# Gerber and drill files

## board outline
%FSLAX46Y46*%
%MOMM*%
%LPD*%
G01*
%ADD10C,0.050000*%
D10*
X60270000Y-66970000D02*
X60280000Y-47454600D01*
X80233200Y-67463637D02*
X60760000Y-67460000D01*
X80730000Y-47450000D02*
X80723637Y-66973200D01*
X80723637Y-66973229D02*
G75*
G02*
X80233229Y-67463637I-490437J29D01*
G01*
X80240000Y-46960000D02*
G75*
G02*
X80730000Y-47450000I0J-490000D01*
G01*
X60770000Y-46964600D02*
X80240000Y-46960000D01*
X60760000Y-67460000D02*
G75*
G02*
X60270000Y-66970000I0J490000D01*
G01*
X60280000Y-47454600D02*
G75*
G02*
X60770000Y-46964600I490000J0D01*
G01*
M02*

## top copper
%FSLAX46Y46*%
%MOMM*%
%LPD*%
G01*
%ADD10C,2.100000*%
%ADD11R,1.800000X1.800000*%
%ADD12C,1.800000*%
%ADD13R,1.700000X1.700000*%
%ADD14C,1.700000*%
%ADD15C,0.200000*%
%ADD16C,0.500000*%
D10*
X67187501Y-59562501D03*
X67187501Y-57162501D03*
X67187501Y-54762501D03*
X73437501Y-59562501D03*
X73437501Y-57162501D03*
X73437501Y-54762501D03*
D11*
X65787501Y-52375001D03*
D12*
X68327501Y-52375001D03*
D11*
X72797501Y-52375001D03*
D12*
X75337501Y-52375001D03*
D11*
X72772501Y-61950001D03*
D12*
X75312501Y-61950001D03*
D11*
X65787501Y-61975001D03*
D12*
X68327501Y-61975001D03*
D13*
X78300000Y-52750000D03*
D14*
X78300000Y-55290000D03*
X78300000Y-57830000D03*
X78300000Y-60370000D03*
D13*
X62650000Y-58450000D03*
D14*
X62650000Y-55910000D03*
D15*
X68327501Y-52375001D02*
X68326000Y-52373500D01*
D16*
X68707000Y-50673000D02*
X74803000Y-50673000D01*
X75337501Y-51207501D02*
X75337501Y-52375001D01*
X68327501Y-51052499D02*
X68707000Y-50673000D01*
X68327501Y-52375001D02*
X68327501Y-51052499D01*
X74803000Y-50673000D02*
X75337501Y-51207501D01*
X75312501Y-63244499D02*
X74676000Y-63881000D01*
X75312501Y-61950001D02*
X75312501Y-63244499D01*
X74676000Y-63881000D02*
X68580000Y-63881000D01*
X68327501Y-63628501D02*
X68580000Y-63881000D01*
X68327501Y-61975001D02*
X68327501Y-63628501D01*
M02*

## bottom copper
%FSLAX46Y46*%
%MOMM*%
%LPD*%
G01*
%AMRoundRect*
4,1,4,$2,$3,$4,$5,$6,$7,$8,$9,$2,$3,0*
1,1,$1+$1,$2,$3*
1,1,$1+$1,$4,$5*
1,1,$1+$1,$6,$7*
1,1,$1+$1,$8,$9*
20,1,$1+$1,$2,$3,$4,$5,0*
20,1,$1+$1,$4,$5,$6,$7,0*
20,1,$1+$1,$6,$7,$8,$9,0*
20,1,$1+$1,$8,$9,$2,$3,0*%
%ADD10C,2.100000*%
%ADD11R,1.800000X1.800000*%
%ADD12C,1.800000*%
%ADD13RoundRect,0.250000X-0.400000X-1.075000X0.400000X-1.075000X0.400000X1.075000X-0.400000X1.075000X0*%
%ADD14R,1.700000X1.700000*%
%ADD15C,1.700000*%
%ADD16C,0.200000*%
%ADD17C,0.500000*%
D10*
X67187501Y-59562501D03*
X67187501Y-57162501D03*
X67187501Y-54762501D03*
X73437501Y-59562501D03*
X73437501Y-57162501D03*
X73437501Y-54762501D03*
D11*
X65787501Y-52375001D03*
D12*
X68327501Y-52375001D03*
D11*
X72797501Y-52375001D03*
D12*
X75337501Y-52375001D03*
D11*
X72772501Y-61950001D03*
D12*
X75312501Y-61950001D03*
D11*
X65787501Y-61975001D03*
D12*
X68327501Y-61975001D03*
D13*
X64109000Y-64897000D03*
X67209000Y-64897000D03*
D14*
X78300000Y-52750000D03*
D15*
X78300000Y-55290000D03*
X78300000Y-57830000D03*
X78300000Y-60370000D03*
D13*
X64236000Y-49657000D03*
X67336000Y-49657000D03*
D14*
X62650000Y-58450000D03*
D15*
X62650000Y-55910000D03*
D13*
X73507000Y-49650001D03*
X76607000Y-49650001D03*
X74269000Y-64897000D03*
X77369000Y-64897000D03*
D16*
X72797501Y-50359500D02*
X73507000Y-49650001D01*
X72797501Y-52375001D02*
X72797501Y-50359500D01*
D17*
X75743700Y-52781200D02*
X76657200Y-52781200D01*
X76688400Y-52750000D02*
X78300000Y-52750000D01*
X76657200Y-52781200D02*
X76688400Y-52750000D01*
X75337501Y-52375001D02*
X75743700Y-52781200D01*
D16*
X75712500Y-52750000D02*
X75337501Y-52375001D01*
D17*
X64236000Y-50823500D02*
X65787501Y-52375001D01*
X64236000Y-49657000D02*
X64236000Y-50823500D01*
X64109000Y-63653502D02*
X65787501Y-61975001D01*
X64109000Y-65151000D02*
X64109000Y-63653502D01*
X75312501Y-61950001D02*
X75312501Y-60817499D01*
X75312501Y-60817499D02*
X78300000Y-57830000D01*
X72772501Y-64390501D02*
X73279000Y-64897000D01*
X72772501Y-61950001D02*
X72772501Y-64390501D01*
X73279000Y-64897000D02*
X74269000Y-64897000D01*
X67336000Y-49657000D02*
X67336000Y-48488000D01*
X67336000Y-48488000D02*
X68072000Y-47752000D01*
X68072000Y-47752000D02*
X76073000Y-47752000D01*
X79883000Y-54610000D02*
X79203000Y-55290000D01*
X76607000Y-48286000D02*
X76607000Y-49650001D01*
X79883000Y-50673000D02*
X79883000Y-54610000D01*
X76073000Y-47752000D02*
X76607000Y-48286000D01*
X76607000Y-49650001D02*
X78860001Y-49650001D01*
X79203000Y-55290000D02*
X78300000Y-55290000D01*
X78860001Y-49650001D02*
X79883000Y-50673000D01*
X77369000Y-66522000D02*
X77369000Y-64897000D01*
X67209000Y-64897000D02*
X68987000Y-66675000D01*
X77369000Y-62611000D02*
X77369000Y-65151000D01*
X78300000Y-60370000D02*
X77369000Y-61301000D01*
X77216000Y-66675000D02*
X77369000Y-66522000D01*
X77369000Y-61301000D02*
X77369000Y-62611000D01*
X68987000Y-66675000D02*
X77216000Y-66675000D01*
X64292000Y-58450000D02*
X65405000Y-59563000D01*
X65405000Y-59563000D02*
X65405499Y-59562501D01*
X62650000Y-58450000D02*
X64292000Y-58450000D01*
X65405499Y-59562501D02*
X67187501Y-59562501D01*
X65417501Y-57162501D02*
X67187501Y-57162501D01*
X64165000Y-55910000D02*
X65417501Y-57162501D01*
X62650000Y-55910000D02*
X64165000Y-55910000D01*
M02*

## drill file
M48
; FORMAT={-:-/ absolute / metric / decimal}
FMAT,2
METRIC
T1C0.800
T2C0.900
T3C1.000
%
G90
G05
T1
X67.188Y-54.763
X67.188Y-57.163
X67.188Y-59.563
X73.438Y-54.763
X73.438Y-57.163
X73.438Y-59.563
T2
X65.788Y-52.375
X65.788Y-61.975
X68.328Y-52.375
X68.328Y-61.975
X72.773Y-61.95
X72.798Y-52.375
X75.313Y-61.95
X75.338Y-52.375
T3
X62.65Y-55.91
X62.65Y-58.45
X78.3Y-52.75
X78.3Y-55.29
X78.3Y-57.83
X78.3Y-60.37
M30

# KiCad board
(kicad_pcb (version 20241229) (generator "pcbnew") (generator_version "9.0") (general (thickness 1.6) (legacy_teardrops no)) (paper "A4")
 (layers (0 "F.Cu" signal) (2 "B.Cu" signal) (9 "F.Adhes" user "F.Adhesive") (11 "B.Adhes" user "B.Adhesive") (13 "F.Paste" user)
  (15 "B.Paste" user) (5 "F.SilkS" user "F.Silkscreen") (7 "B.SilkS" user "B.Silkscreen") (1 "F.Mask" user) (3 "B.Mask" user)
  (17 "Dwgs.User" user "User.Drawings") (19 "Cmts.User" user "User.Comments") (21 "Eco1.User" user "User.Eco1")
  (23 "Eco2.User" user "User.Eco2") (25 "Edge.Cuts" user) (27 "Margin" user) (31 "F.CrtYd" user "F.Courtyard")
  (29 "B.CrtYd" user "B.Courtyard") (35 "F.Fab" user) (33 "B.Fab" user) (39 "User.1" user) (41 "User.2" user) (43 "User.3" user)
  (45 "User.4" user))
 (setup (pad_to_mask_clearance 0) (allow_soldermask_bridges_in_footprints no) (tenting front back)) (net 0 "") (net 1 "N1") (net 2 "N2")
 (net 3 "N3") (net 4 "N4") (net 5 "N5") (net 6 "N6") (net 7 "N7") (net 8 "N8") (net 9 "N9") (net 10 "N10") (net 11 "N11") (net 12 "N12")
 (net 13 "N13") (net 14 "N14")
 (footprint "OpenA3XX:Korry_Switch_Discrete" (layer "F.Cu") (at 76.287501 61.262501)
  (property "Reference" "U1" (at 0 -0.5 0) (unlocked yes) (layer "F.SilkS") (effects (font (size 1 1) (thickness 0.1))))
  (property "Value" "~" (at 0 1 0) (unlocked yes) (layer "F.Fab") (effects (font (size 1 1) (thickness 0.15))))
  (pad "1" thru_hole circle (at -9.1 -1.7) (size 2.1 2.1) (drill 0.8) (layers "*.Cu" "*.Mask") (remove_unused_layers no) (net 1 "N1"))
  (pad "2" thru_hole circle (at -9.1 -4.1) (size 2.1 2.1) (drill 0.8) (layers "*.Cu" "*.Mask") (remove_unused_layers no) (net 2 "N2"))
  (pad "3" thru_hole circle (at -9.1 -6.5) (size 2.1 2.1) (drill 0.8) (layers "*.Cu" "*.Mask") (remove_unused_layers no) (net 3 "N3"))
  (pad "4" thru_hole circle (at -2.85 -1.7) (size 2.1 2.1) (drill 0.8) (layers "*.Cu" "*.Mask") (remove_unused_layers no) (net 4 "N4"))
  (pad "5" thru_hole circle (at -2.85 -4.1) (size 2.1 2.1) (drill 0.8) (layers "*.Cu" "*.Mask") (remove_unused_layers no) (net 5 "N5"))
  (pad "6" thru_hole circle (at -2.85 -6.5) (size 2.1 2.1) (drill 0.8) (layers "*.Cu" "*.Mask") (remove_unused_layers no) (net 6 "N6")))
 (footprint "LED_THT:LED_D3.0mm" (layer "F.Cu") (at 65.787501 52.375001)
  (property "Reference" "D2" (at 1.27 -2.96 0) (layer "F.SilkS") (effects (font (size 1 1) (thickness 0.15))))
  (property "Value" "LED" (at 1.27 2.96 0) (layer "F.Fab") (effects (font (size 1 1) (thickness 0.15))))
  (pad "1" thru_hole rect (at 0 0) (size 1.8 1.8) (drill 0.9) (layers "*.Cu" "*.Mask") (remove_unused_layers no) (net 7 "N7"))
  (pad "2" thru_hole circle (at 2.54 0) (size 1.8 1.8) (drill 0.9) (layers "*.Cu" "*.Mask") (remove_unused_layers no) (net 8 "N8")))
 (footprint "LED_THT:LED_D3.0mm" (layer "F.Cu") (at 72.797501 52.375001)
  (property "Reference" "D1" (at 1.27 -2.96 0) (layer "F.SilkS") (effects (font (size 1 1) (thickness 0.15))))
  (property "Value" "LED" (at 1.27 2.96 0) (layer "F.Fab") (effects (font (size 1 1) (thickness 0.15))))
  (pad "1" thru_hole rect (at 0 0) (size 1.8 1.8) (drill 0.9) (layers "*.Cu" "*.Mask") (remove_unused_layers no) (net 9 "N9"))
  (pad "2" thru_hole circle (at 2.54 0) (size 1.8 1.8) (drill 0.9) (layers "*.Cu" "*.Mask") (remove_unused_layers no) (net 8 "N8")))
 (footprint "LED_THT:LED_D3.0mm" (layer "F.Cu") (at 72.772501 61.950001)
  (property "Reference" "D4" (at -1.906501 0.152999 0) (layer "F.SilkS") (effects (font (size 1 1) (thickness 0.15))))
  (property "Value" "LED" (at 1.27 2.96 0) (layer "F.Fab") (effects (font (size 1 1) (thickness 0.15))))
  (pad "1" thru_hole rect (at 0 0) (size 1.8 1.8) (drill 0.9) (layers "*.Cu" "*.Mask") (remove_unused_layers no) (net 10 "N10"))
  (pad "2" thru_hole circle (at 2.54 0) (size 1.8 1.8) (drill 0.9) (layers "*.Cu" "*.Mask") (remove_unused_layers no) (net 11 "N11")))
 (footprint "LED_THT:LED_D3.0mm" (layer "F.Cu") (at 65.787501 61.975001)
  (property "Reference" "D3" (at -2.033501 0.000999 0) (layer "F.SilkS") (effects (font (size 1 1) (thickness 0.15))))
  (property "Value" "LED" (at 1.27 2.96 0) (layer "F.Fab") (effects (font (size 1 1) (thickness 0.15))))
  (pad "1" thru_hole rect (at 0 0) (size 1.8 1.8) (drill 0.9) (layers "*.Cu" "*.Mask") (remove_unused_layers no) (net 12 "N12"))
  (pad "2" thru_hole circle (at 2.54 0) (size 1.8 1.8) (drill 0.9) (layers "*.Cu" "*.Mask") (remove_unused_layers no) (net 11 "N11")))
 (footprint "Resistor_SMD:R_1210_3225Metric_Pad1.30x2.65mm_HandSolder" (layer "B.Cu") (at 65.659 64.897)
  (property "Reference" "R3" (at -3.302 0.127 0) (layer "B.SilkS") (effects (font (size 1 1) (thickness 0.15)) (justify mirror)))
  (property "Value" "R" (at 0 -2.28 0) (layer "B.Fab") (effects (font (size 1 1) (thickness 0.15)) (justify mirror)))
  (pad "1" smd roundrect (at -1.55 0) (size 1.3 2.65) (layers "B.Cu" "B.Mask" "B.Paste") (roundrect_rratio 0.192308) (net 12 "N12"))
  (pad "2" smd roundrect (at 1.55 0) (size 1.3 2.65) (layers "B.Cu" "B.Mask" "B.Paste") (roundrect_rratio 0.192308) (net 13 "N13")))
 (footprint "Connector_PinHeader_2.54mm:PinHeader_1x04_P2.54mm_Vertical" (layer "B.Cu") (at 78.3 52.75 180)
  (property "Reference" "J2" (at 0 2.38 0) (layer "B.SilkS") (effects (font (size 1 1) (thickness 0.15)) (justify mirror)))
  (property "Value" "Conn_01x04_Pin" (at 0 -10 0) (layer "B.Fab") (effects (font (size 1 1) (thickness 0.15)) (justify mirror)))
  (pad "1" thru_hole rect (at 0 0 180) (size 1.7 1.7) (drill 1) (layers "*.Cu" "*.Mask") (remove_unused_layers no) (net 8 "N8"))
  (pad "2" thru_hole circle (at 0 -2.54 180) (size 1.7 1.7) (drill 1) (layers "*.Cu" "*.Mask") (remove_unused_layers no) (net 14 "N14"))
  (pad "3" thru_hole circle (at 0 -5.08 180) (size 1.7 1.7) (drill 1) (layers "*.Cu" "*.Mask") (remove_unused_layers no) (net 11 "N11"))
  (pad "4" thru_hole circle (at 0 -7.62 180) (size 1.7 1.7) (drill 1) (layers "*.Cu" "*.Mask") (remove_unused_layers no) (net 13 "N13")))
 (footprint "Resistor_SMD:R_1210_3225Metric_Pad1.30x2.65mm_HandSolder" (layer "B.Cu") (at 65.786 49.657)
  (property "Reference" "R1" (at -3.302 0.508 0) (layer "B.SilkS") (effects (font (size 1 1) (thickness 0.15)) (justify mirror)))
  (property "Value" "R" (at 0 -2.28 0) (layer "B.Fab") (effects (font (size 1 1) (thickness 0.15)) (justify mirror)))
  (pad "1" smd roundrect (at -1.55 0) (size 1.3 2.65) (layers "B.Cu" "B.Mask" "B.Paste") (roundrect_rratio 0.192308) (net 7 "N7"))
  (pad "2" smd roundrect (at 1.55 0) (size 1.3 2.65) (layers "B.Cu" "B.Mask" "B.Paste") (roundrect_rratio 0.192308) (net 14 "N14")))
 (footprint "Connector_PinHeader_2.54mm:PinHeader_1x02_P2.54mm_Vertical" (layer "B.Cu") (at 62.65 58.45)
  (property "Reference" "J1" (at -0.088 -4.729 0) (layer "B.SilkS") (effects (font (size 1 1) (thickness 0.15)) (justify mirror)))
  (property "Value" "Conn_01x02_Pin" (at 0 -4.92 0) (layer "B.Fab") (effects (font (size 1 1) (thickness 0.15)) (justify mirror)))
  (pad "1" thru_hole rect (at 0 0) (size 1.7 1.7) (drill 1) (layers "*.Cu" "*.Mask") (remove_unused_layers no) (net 1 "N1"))
  (pad "2" thru_hole circle (at 0 -2.54) (size 1.7 1.7) (drill 1) (layers "*.Cu" "*.Mask") (remove_unused_layers no) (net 2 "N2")))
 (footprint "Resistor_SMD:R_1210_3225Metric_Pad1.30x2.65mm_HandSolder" (layer "B.Cu") (at 75.057 49.650001)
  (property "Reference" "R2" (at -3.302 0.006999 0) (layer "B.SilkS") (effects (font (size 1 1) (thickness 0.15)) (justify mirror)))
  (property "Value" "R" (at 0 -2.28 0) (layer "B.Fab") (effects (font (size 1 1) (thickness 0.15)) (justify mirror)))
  (pad "1" smd roundrect (at -1.55 0) (size 1.3 2.65) (layers "B.Cu" "B.Mask" "B.Paste") (roundrect_rratio 0.192308) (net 9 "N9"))
  (pad "2" smd roundrect (at 1.55 0) (size 1.3 2.65) (layers "B.Cu" "B.Mask" "B.Paste") (roundrect_rratio 0.192308) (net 14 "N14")))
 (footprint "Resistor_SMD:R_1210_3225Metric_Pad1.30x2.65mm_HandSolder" (layer "B.Cu") (at 75.819 64.897)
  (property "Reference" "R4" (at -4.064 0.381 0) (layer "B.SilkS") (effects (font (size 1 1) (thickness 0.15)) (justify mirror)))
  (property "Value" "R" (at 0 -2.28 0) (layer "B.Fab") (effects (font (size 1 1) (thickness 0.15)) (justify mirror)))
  (pad "1" smd roundrect (at -1.55 0) (size 1.3 2.65) (layers "B.Cu" "B.Mask" "B.Paste") (roundrect_rratio 0.192308) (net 10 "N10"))
  (pad "2" smd roundrect (at 1.55 0) (size 1.3 2.65) (layers "B.Cu" "B.Mask" "B.Paste") (roundrect_rratio 0.192308) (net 13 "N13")))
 (gr_line (start 60.27 66.97) (end 60.28 47.4546) (stroke (width 0.05) (type default)) (layer "Edge.Cuts"))
 (gr_line (start 80.2332 67.463637) (end 60.76 67.46) (stroke (width 0.05) (type default)) (layer "Edge.Cuts"))
 (gr_line (start 80.73 47.45) (end 80.723637 66.9732) (stroke (width 0.05) (type default)) (layer "Edge.Cuts"))
 (gr_arc (start 80.723637 66.973229) (mid 80.58 67.32) (end 80.233229 67.463637) (stroke (width 0.05) (type default)) (layer "Edge.Cuts"))
 (gr_arc (start 80.24 46.96) (mid 80.586482 47.103518) (end 80.73 47.45) (stroke (width 0.05) (type default)) (layer "Edge.Cuts"))
 (gr_line (start 60.77 46.9646) (end 80.24 46.96) (stroke (width 0.05) (type default)) (layer "Edge.Cuts"))
 (gr_arc (start 60.76 67.46) (mid 60.413518 67.316482) (end 60.27 66.97) (stroke (width 0.05) (type default)) (layer "Edge.Cuts"))
 (gr_arc (start 60.28 47.4546) (mid 60.423518 47.108118) (end 60.77 46.9646) (stroke (width 0.05) (type default)) (layer "Edge.Cuts"))
 (segment (start 72.797501 50.3595) (end 73.507 49.650001) (width 0.2) (layer "B.Cu") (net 9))
 (segment (start 72.797501 52.375001) (end 72.797501 50.3595) (width 0.2) (layer "B.Cu") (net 9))
 (segment (start 68.327501 52.375001) (end 68.326 52.3735) (width 0.2) (layer "F.Cu") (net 8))
 (segment (start 68.707 50.673) (end 74.803 50.673) (width 0.5) (layer "F.Cu") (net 8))
 (segment (start 75.337501 51.207501) (end 75.337501 52.375001) (width 0.5) (layer "F.Cu") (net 8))
 (segment (start 68.327501 51.052499) (end 68.707 50.673) (width 0.5) (layer "F.Cu") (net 8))
 (segment (start 68.327501 52.375001) (end 68.327501 51.052499) (width 0.5) (layer "F.Cu") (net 8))
 (segment (start 74.803 50.673) (end 75.337501 51.207501) (width 0.5) (layer "F.Cu") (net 8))
 (segment (start 75.7437 52.7812) (end 76.6572 52.7812) (width 0.5) (layer "B.Cu") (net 8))
 (segment (start 76.6884 52.75) (end 78.3 52.75) (width 0.5) (layer "B.Cu") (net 8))
 (segment (start 76.6572 52.7812) (end 76.6884 52.75) (width 0.5) (layer "B.Cu") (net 8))
 (segment (start 75.337501 52.375001) (end 75.7437 52.7812) (width 0.5) (layer "B.Cu") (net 8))
 (segment (start 75.7125 52.75) (end 75.337501 52.375001) (width 0.2) (layer "B.Cu") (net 8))
 (segment (start 64.236 50.8235) (end 65.787501 52.375001) (width 0.5) (layer "B.Cu") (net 7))
 (segment (start 64.236 49.657) (end 64.236 50.8235) (width 0.5) (layer "B.Cu") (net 7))
 (segment (start 64.109 63.653502) (end 65.787501 61.975001) (width 0.5) (layer "B.Cu") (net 12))
 (segment (start 64.109 65.151) (end 64.109 63.653502) (width 0.5) (layer "B.Cu") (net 12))
 (segment (start 75.312501 63.244499) (end 74.676 63.881) (width 0.5) (layer "F.Cu") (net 11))
 (segment (start 75.312501 61.950001) (end 75.312501 63.244499) (width 0.5) (layer "F.Cu") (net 11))
 (segment (start 74.676 63.881) (end 68.58 63.881) (width 0.5) (layer "F.Cu") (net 11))
 (segment (start 68.327501 63.628501) (end 68.58 63.881) (width 0.5) (layer "F.Cu") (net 11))
 (segment (start 68.327501 61.975001) (end 68.327501 63.628501) (width 0.5) (layer "F.Cu") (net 11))
 (segment (start 75.312501 61.950001) (end 75.312501 60.817499) (width 0.5) (layer "B.Cu") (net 11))
 (segment (start 75.312501 60.817499) (end 78.3 57.83) (width 0.5) (layer "B.Cu") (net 11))
 (segment (start 72.772501 64.390501) (end 73.279 64.897) (width 0.5) (layer "B.Cu") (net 10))
 (segment (start 72.772501 61.950001) (end 72.772501 64.390501) (width 0.5) (layer "B.Cu") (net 10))
 (segment (start 73.279 64.897) (end 74.269 64.897) (width 0.5) (layer "B.Cu") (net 10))
 (segment (start 67.336 49.657) (end 67.336 48.488) (width 0.5) (layer "B.Cu") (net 14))
 (segment (start 67.336 48.488) (end 68.072 47.752) (width 0.5) (layer "B.Cu") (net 14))
 (segment (start 68.072 47.752) (end 76.073 47.752) (width 0.5) (layer "B.Cu") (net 14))
 (segment (start 79.883 54.61) (end 79.203 55.29) (width 0.5) (layer "B.Cu") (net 14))
 (segment (start 76.607 48.286) (end 76.607 49.650001) (width 0.5) (layer "B.Cu") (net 14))
 (segment (start 79.883 50.673) (end 79.883 54.61) (width 0.5) (layer "B.Cu") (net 14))
 (segment (start 76.073 47.752) (end 76.607 48.286) (width 0.5) (layer "B.Cu") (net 14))
 (segment (start 76.607 49.650001) (end 78.860001 49.650001) (width 0.5) (layer "B.Cu") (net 14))
 (segment (start 79.203 55.29) (end 78.3 55.29) (width 0.5) (layer "B.Cu") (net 14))
 (segment (start 78.860001 49.650001) (end 79.883 50.673) (width 0.5) (layer "B.Cu") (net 14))
 (segment (start 77.369 66.522) (end 77.369 64.897) (width 0.5) (layer "B.Cu") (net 13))
 (segment (start 67.209 64.897) (end 68.987 66.675) (width 0.5) (layer "B.Cu") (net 13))
 (segment (start 77.369 62.611) (end 77.369 65.151) (width 0.5) (layer "B.Cu") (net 13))
 (segment (start 78.3 60.37) (end 77.369 61.301) (width 0.5) (layer "B.Cu") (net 13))
 (segment (start 77.216 66.675) (end 77.369 66.522) (width 0.5) (layer "B.Cu") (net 13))
 (segment (start 77.369 61.301) (end 77.369 62.611) (width 0.5) (layer "B.Cu") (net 13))
 (segment (start 68.987 66.675) (end 77.216 66.675) (width 0.5) (layer "B.Cu") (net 13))
 (segment (start 64.292 58.45) (end 65.405 59.563) (width 0.5) (layer "B.Cu") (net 1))
 (segment (start 65.405 59.563) (end 65.405499 59.562501) (width 0.5) (layer "B.Cu") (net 1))
 (segment (start 62.65 58.45) (end 64.292 58.45) (width 0.5) (layer "B.Cu") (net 1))
 (segment (start 65.405499 59.562501) (end 67.187501 59.562501) (width 0.5) (layer "B.Cu") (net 1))
 (segment (start 65.417501 57.162501) (end 67.187501 57.162501) (width 0.5) (layer "B.Cu") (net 2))
 (segment (start 64.165 55.91) (end 65.417501 57.162501) (width 0.5) (layer "B.Cu") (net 2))
 (segment (start 62.65 55.91) (end 64.165 55.91) (width 0.5) (layer "B.Cu") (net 2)))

